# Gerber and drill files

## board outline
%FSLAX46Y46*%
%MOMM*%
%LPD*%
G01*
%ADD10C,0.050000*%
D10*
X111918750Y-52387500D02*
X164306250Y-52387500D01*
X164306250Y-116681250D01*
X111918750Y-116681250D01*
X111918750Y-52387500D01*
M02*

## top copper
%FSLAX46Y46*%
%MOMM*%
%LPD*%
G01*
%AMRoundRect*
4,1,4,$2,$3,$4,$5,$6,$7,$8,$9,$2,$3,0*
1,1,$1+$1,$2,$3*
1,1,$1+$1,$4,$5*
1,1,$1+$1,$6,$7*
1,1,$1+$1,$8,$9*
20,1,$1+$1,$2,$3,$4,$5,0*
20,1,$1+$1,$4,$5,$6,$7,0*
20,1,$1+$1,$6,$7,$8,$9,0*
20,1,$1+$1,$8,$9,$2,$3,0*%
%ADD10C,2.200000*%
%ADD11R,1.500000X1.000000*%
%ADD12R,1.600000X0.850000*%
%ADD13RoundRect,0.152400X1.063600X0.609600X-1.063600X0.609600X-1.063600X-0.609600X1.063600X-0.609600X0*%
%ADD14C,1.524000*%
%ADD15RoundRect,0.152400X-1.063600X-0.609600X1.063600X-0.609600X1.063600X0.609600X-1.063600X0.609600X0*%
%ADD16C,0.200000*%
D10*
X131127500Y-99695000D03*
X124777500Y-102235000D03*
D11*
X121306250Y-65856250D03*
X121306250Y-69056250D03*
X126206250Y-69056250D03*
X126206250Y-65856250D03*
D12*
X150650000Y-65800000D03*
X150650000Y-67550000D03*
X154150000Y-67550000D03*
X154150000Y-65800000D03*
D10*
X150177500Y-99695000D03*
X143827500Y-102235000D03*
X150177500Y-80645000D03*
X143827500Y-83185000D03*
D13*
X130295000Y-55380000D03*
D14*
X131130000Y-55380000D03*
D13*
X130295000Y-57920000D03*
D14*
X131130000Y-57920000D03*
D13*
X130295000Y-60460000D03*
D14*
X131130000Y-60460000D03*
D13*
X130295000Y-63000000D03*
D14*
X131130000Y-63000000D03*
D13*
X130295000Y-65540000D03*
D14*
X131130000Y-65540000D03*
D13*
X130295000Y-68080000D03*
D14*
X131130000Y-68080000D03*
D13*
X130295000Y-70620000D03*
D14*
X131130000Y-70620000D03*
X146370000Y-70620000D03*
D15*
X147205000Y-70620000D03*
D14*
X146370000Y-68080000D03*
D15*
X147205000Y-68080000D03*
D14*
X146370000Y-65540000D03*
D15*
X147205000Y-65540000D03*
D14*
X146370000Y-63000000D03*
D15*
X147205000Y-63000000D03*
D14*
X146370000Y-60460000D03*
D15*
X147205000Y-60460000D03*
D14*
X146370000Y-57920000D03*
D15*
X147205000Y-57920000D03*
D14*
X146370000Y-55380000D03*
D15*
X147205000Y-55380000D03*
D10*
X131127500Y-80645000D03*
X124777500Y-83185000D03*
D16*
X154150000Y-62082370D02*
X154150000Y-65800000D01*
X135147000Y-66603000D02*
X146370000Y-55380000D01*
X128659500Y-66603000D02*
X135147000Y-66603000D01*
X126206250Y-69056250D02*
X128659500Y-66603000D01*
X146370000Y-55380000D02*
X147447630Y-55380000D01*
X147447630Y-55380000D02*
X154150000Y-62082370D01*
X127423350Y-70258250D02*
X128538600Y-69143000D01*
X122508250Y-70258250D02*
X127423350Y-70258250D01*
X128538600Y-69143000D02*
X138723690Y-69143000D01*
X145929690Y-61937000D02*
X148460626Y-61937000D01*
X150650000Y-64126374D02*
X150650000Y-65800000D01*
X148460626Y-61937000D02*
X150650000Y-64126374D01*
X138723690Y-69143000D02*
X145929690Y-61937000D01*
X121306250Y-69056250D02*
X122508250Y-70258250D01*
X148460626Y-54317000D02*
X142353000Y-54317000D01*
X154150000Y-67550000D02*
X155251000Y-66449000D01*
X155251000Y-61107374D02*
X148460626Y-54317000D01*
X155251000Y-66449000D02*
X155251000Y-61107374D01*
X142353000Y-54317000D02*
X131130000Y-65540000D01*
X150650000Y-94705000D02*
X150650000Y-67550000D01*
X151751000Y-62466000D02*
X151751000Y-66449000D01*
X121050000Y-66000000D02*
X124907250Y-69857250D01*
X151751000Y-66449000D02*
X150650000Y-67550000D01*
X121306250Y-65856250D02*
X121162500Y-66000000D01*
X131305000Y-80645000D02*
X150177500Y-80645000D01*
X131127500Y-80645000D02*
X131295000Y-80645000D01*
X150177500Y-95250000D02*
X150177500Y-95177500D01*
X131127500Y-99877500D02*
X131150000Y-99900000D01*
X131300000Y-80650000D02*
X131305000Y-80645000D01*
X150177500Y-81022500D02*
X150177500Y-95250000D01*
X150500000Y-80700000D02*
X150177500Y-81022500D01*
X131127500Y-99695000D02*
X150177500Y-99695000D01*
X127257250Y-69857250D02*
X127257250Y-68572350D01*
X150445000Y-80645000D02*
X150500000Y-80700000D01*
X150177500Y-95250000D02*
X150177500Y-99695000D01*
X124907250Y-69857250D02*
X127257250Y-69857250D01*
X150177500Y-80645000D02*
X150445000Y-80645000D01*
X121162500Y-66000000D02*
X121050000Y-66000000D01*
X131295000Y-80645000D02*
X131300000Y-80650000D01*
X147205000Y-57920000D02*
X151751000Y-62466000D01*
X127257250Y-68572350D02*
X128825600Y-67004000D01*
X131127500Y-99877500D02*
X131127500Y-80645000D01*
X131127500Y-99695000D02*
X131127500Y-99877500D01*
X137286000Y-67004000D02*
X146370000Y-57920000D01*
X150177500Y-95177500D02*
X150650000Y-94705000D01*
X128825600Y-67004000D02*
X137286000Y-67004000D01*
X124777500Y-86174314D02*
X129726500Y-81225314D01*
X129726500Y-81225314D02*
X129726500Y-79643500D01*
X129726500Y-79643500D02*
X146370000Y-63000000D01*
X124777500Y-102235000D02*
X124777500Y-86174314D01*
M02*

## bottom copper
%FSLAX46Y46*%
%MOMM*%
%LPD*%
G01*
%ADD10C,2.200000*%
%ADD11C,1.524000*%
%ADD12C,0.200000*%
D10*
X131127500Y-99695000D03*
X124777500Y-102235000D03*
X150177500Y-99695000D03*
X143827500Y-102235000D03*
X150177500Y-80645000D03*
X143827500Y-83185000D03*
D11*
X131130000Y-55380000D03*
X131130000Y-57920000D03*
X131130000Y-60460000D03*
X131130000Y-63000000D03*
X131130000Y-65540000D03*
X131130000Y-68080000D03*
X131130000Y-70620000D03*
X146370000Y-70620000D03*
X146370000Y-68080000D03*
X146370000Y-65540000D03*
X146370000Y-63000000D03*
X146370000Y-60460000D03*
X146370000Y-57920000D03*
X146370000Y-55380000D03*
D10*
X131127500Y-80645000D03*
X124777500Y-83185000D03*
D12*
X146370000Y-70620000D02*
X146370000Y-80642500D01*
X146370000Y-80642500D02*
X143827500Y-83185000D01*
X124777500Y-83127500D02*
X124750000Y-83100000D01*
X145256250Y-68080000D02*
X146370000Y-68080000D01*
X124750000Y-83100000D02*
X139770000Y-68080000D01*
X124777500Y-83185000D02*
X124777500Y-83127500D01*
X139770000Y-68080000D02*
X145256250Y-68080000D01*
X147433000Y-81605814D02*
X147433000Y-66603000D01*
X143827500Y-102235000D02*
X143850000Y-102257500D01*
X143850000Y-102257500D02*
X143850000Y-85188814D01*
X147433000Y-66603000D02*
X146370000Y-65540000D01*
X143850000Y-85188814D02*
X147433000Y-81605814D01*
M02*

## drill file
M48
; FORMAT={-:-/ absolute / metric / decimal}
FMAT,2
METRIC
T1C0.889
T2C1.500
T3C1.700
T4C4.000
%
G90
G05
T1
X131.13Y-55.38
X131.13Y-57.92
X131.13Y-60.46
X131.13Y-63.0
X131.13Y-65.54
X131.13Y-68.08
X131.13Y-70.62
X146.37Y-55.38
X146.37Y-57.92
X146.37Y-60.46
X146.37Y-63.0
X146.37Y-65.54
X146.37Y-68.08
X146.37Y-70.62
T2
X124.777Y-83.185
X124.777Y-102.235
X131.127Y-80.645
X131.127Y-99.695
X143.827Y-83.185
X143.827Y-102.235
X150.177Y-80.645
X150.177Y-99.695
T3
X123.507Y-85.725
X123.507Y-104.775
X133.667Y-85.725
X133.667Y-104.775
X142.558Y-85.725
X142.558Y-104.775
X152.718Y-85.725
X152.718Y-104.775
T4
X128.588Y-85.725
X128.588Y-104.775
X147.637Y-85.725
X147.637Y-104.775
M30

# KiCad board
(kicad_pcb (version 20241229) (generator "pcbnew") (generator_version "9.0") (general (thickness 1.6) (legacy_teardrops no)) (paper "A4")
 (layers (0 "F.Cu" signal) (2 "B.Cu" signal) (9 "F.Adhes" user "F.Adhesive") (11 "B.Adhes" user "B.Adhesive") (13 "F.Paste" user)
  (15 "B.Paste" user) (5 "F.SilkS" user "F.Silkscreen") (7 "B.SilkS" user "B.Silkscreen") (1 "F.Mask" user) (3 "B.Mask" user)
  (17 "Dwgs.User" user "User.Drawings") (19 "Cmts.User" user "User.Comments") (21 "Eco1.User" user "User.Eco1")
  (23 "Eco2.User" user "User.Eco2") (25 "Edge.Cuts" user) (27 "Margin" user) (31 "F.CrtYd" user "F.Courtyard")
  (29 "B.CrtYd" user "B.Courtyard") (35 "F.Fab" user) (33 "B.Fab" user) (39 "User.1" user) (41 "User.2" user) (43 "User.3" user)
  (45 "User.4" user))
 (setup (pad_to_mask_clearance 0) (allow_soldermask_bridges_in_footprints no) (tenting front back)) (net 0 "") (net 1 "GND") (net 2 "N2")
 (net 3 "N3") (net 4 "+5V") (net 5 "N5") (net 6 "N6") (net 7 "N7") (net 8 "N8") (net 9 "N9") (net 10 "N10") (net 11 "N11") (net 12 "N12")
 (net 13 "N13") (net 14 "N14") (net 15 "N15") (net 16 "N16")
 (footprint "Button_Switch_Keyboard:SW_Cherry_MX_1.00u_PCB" (layer "F.Cu") (at 131.1275 99.695)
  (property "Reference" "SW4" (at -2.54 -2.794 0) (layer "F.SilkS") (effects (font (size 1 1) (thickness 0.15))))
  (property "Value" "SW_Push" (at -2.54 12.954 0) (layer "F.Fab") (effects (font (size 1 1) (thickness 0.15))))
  (pad "" np_thru_hole circle (at -7.62 5.08) (size 1.7 1.7) (drill 1.7) (layers "*.Cu" "*.Mask"))
  (pad "" np_thru_hole circle (at -2.54 5.08) (size 4 4) (drill 4) (layers "*.Cu" "*.Mask"))
  (pad "" np_thru_hole circle (at 2.54 5.08) (size 1.7 1.7) (drill 1.7) (layers "*.Cu" "*.Mask"))
  (pad "1" thru_hole circle (at 0 0) (size 2.2 2.2) (drill 1.5) (layers "*.Cu" "*.Mask") (remove_unused_layers no) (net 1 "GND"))
  (pad "2" thru_hole circle (at -6.35 2.54) (size 2.2 2.2) (drill 1.5) (layers "*.Cu" "*.Mask") (remove_unused_layers no) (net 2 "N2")))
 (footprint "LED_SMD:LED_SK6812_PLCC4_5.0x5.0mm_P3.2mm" (layer "F.Cu") (at 123.75625 67.45625)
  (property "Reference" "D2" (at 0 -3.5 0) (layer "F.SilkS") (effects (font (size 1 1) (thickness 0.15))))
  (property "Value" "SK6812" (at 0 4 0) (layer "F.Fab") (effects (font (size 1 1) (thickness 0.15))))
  (pad "1" smd rect (at -2.45 -1.6 180) (size 1.5 1) (layers "F.Cu" "F.Mask" "F.Paste") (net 1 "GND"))
  (pad "2" smd rect (at -2.45 1.6 180) (size 1.5 1) (layers "F.Cu" "F.Mask" "F.Paste") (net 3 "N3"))
  (pad "3" smd rect (at 2.45 1.6 180) (size 1.5 1) (layers "F.Cu" "F.Mask" "F.Paste") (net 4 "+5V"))
  (pad "4" smd rect (at 2.45 -1.6 180) (size 1.5 1) (layers "F.Cu" "F.Mask" "F.Paste") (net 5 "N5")))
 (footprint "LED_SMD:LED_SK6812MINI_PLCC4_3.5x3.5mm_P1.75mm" (layer "F.Cu") (at 152.4 66.675)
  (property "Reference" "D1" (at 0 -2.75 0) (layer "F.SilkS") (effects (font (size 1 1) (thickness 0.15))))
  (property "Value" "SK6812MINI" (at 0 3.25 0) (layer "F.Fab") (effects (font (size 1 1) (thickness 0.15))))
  (pad "1" smd rect (at -1.75 -0.875) (size 1.6 0.85) (layers "F.Cu" "F.Mask" "F.Paste") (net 3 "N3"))
  (pad "2" smd rect (at -1.75 0.875) (size 1.6 0.85) (layers "F.Cu" "F.Mask" "F.Paste") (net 1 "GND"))
  (pad "3" smd rect (at 1.75 0.875) (size 1.6 0.85) (layers "F.Cu" "F.Mask" "F.Paste") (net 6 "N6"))
  (pad "4" smd rect (at 1.75 -0.875) (size 1.6 0.85) (layers "F.Cu" "F.Mask" "F.Paste") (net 4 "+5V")))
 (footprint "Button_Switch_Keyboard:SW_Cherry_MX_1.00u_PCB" (layer "F.Cu") (at 150.1775 99.695)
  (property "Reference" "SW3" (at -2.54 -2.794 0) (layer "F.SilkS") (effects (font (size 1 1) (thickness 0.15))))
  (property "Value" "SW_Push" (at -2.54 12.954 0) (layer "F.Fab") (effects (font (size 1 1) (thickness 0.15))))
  (pad "" np_thru_hole circle (at -7.62 5.08) (size 1.7 1.7) (drill 1.7) (layers "*.Cu" "*.Mask"))
  (pad "" np_thru_hole circle (at -2.54 5.08) (size 4 4) (drill 4) (layers "*.Cu" "*.Mask"))
  (pad "" np_thru_hole circle (at 2.54 5.08) (size 1.7 1.7) (drill 1.7) (layers "*.Cu" "*.Mask"))
  (pad "1" thru_hole circle (at 0 0) (size 2.2 2.2) (drill 1.5) (layers "*.Cu" "*.Mask") (remove_unused_layers no) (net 1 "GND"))
  (pad "2" thru_hole circle (at -6.35 2.54) (size 2.2 2.2) (drill 1.5) (layers "*.Cu" "*.Mask") (remove_unused_layers no) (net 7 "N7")))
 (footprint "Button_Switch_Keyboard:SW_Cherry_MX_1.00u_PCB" (layer "F.Cu") (at 150.1775 80.645)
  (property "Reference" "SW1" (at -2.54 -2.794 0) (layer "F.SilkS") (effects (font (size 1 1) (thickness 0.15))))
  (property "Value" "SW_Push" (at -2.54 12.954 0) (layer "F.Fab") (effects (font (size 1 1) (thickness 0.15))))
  (pad "" np_thru_hole circle (at -7.62 5.08) (size 1.7 1.7) (drill 1.7) (layers "*.Cu" "*.Mask"))
  (pad "" np_thru_hole circle (at -2.54 5.08) (size 4 4) (drill 4) (layers "*.Cu" "*.Mask"))
  (pad "" np_thru_hole circle (at 2.54 5.08) (size 1.7 1.7) (drill 1.7) (layers "*.Cu" "*.Mask"))
  (pad "1" thru_hole circle (at 0 0) (size 2.2 2.2) (drill 1.5) (layers "*.Cu" "*.Mask") (remove_unused_layers no) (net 1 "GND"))
  (pad "2" thru_hole circle (at -6.35 2.54) (size 2.2 2.2) (drill 1.5) (layers "*.Cu" "*.Mask") (remove_unused_layers no) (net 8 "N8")))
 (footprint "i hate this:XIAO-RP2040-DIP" (layer "F.Cu") (at 138.75 63)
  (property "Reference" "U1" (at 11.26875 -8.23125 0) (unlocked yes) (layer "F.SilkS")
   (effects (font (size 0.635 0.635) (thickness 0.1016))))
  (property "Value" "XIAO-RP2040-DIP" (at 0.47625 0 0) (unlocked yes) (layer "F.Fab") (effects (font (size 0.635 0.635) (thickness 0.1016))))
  (pad "1" smd roundrect (at -8.455 -7.62 180) (size 2.432 1.524) (layers "F.Cu" "F.Mask") (roundrect_rratio 0.1) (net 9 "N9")
   (thermal_bridge_angle 45))
  (pad "1" thru_hole circle (at -7.62 -7.62 180) (size 1.524 1.524) (drill 0.889) (layers "*.Cu" "*.Mask") (remove_unused_layers no)
   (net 9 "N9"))
  (pad "2" smd roundrect (at -8.455 -5.08 180) (size 2.432 1.524) (layers "F.Cu" "F.Mask") (roundrect_rratio 0.1) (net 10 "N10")
   (thermal_bridge_angle 45))
  (pad "2" thru_hole circle (at -7.62 -5.08 180) (size 1.524 1.524) (drill 0.889) (layers "*.Cu" "*.Mask") (remove_unused_layers no)
   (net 10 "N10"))
  (pad "3" smd roundrect (at -8.455 -2.54 180) (size 2.432 1.524) (layers "F.Cu" "F.Mask") (roundrect_rratio 0.1) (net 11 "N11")
   (thermal_bridge_angle 45))
  (pad "3" thru_hole circle (at -7.62 -2.54 180) (size 1.524 1.524) (drill 0.889) (layers "*.Cu" "*.Mask") (remove_unused_layers no)
   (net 11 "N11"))
  (pad "4" smd roundrect (at -8.455 0 180) (size 2.432 1.524) (layers "F.Cu" "F.Mask") (roundrect_rratio 0.1) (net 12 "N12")
   (thermal_bridge_angle 45))
  (pad "4" thru_hole circle (at -7.62 0 180) (size 1.524 1.524) (drill 0.889) (layers "*.Cu" "*.Mask") (remove_unused_layers no)
   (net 12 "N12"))
  (pad "5" smd roundrect (at -8.455 2.54 180) (size 2.432 1.524) (layers "F.Cu" "F.Mask") (roundrect_rratio 0.1) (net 6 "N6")
   (thermal_bridge_angle 45))
  (pad "5" thru_hole circle (at -7.62 2.54 180) (size 1.524 1.524) (drill 0.889) (layers "*.Cu" "*.Mask") (remove_unused_layers no)
   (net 6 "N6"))
  (pad "6" smd roundrect (at -8.455 5.08 180) (size 2.432 1.524) (layers "F.Cu" "F.Mask") (roundrect_rratio 0.1) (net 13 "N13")
   (thermal_bridge_angle 45))
  (pad "6" thru_hole circle (at -7.62 5.08 180) (size 1.524 1.524) (drill 0.889) (layers "*.Cu" "*.Mask") (remove_unused_layers no)
   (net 13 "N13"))
  (pad "7" smd roundrect (at -8.455 7.62 180) (size 2.432 1.524) (layers "F.Cu" "F.Mask") (roundrect_rratio 0.1) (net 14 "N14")
   (thermal_bridge_angle 45))
  (pad "7" thru_hole circle (at -7.62 7.62 180) (size 1.524 1.524) (drill 0.889) (layers "*.Cu" "*.Mask") (remove_unused_layers no)
   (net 14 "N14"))
  (pad "8" thru_hole circle (at 7.62 7.62) (size 1.524 1.524) (drill 0.889) (layers "*.Cu" "*.Mask") (remove_unused_layers no) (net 8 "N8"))
  (pad "8" smd roundrect (at 8.455 7.62) (size 2.432 1.524) (layers "F.Cu" "F.Mask") (roundrect_rratio 0.1) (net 8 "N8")
   (thermal_bridge_angle 45))
  (pad "9" thru_hole circle (at 7.62 5.08) (size 1.524 1.524) (drill 0.889) (layers "*.Cu" "*.Mask") (remove_unused_layers no)
   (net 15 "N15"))
  (pad "9" smd roundrect (at 8.455 5.08) (size 2.432 1.524) (layers "F.Cu" "F.Mask") (roundrect_rratio 0.1) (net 15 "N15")
   (thermal_bridge_angle 45))
  (pad "10" thru_hole circle (at 7.62 2.54) (size 1.524 1.524) (drill 0.889) (layers "*.Cu" "*.Mask") (remove_unused_layers no) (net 7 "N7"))
  (pad "10" smd roundrect (at 8.455 2.54) (size 2.432 1.524) (layers "F.Cu" "F.Mask") (roundrect_rratio 0.1) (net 7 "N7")
   (thermal_bridge_angle 45))
  (pad "11" thru_hole circle (at 7.62 0) (size 1.524 1.524) (drill 0.889) (layers "*.Cu" "*.Mask") (remove_unused_layers no) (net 2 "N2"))
  (pad "11" smd roundrect (at 8.455 0) (size 2.432 1.524) (layers "F.Cu" "F.Mask") (roundrect_rratio 0.1) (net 2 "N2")
   (thermal_bridge_angle 45))
  (pad "12" thru_hole circle (at 7.62 -2.54) (size 1.524 1.524) (drill 0.889) (layers "*.Cu" "*.Mask") (remove_unused_layers no)
   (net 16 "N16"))
  (pad "12" smd roundrect (at 8.455 -2.54) (size 2.432 1.524) (layers "F.Cu" "F.Mask") (roundrect_rratio 0.1) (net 16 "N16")
   (thermal_bridge_angle 45))
  (pad "13" thru_hole circle (at 7.62 -5.08) (size 1.524 1.524) (drill 0.889) (layers "*.Cu" "*.Mask") (remove_unused_layers no)
   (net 1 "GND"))
  (pad "13" smd roundrect (at 8.455 -5.08) (size 2.432 1.524) (layers "F.Cu" "F.Mask") (roundrect_rratio 0.1) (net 1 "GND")
   (thermal_bridge_angle 45))
  (pad "14" thru_hole circle (at 7.62 -7.62) (size 1.524 1.524) (drill 0.889) (layers "*.Cu" "*.Mask") (remove_unused_layers no)
   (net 4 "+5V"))
  (pad "14" smd roundrect (at 8.455 -7.62) (size 2.432 1.524) (layers "F.Cu" "F.Mask") (roundrect_rratio 0.1) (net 4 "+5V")
   (thermal_bridge_angle 45)))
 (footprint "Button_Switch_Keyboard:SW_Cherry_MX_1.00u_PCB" (layer "F.Cu") (at 131.1275 80.645)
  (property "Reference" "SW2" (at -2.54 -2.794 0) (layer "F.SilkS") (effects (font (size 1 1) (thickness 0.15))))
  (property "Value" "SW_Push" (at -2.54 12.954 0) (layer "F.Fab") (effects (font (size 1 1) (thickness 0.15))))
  (pad "" np_thru_hole circle (at -7.62 5.08) (size 1.7 1.7) (drill 1.7) (layers "*.Cu" "*.Mask"))
  (pad "" np_thru_hole circle (at -2.54 5.08) (size 4 4) (drill 4) (layers "*.Cu" "*.Mask"))
  (pad "" np_thru_hole circle (at 2.54 5.08) (size 1.7 1.7) (drill 1.7) (layers "*.Cu" "*.Mask"))
  (pad "1" thru_hole circle (at 0 0) (size 2.2 2.2) (drill 1.5) (layers "*.Cu" "*.Mask") (remove_unused_layers no) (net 1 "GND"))
  (pad "2" thru_hole circle (at -6.35 2.54) (size 2.2 2.2) (drill 1.5) (layers "*.Cu" "*.Mask") (remove_unused_layers no) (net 15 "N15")))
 (gr_rect (start 111.91875 52.3875) (end 164.30625 116.68125) (stroke (width 0.05) (type default)) (fill no) (layer "Edge.Cuts"))
 (segment (start 154.15 62.08237) (end 154.15 65.8) (width 0.2) (layer "F.Cu") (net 4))
 (segment (start 135.147 66.603) (end 146.37 55.38) (width 0.2) (layer "F.Cu") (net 4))
 (segment (start 128.6595 66.603) (end 135.147 66.603) (width 0.2) (layer "F.Cu") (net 4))
 (segment (start 126.20625 69.05625) (end 128.6595 66.603) (width 0.2) (layer "F.Cu") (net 4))
 (segment (start 146.37 55.38) (end 147.44763 55.38) (width 0.2) (layer "F.Cu") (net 4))
 (segment (start 147.44763 55.38) (end 154.15 62.08237) (width 0.2) (layer "F.Cu") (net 4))
 (segment (start 127.42335 70.25825) (end 128.5386 69.143) (width 0.2) (layer "F.Cu") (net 3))
 (segment (start 122.50825 70.25825) (end 127.42335 70.25825) (width 0.2) (layer "F.Cu") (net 3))
 (segment (start 128.5386 69.143) (end 138.72369 69.143) (width 0.2) (layer "F.Cu") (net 3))
 (segment (start 145.92969 61.937) (end 148.460626 61.937) (width 0.2) (layer "F.Cu") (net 3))
 (segment (start 150.65 64.126374) (end 150.65 65.8) (width 0.2) (layer "F.Cu") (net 3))
 (segment (start 148.460626 61.937) (end 150.65 64.126374) (width 0.2) (layer "F.Cu") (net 3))
 (segment (start 138.72369 69.143) (end 145.92969 61.937) (width 0.2) (layer "F.Cu") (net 3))
 (segment (start 121.30625 69.05625) (end 122.50825 70.25825) (width 0.2) (layer "F.Cu") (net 3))
 (segment (start 148.460626 54.317) (end 142.353 54.317) (width 0.2) (layer "F.Cu") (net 6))
 (segment (start 154.15 67.55) (end 155.251 66.449) (width 0.2) (layer "F.Cu") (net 6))
 (segment (start 155.251 61.107374) (end 148.460626 54.317) (width 0.2) (layer "F.Cu") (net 6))
 (segment (start 155.251 66.449) (end 155.251 61.107374) (width 0.2) (layer "F.Cu") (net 6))
 (segment (start 142.353 54.317) (end 131.13 65.54) (width 0.2) (layer "F.Cu") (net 6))
 (segment (start 150.65 94.705) (end 150.65 67.55) (width 0.2) (layer "F.Cu") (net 1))
 (segment (start 151.751 62.466) (end 151.751 66.449) (width 0.2) (layer "F.Cu") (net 1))
 (segment (start 121.05 66) (end 124.90725 69.85725) (width 0.2) (layer "F.Cu") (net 1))
 (segment (start 151.751 66.449) (end 150.65 67.55) (width 0.2) (layer "F.Cu") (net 1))
 (segment (start 121.30625 65.85625) (end 121.1625 66) (width 0.2) (layer "F.Cu") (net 1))
 (segment (start 131.305 80.645) (end 150.1775 80.645) (width 0.2) (layer "F.Cu") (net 1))
 (segment (start 131.1275 80.645) (end 131.295 80.645) (width 0.2) (layer "F.Cu") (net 1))
 (segment (start 150.1775 95.25) (end 150.1775 95.1775) (width 0.2) (layer "F.Cu") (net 1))
 (segment (start 131.1275 99.8775) (end 131.15 99.9) (width 0.2) (layer "F.Cu") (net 1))
 (segment (start 131.3 80.65) (end 131.305 80.645) (width 0.2) (layer "F.Cu") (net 1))
 (segment (start 150.1775 81.0225) (end 150.1775 95.25) (width 0.2) (layer "F.Cu") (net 1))
 (segment (start 150.5 80.7) (end 150.1775 81.0225) (width 0.2) (layer "F.Cu") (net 1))
 (segment (start 131.1275 99.695) (end 150.1775 99.695) (width 0.2) (layer "F.Cu") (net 1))
 (segment (start 127.25725 69.85725) (end 127.25725 68.57235) (width 0.2) (layer "F.Cu") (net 1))
 (segment (start 150.445 80.645) (end 150.5 80.7) (width 0.2) (layer "F.Cu") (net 1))
 (segment (start 150.1775 95.25) (end 150.1775 99.695) (width 0.2) (layer "F.Cu") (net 1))
 (segment (start 124.90725 69.85725) (end 127.25725 69.85725) (width 0.2) (layer "F.Cu") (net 1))
 (segment (start 150.1775 80.645) (end 150.445 80.645) (width 0.2) (layer "F.Cu") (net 1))
 (segment (start 121.1625 66) (end 121.05 66) (width 0.2) (layer "F.Cu") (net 1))
 (segment (start 131.295 80.645) (end 131.3 80.65) (width 0.2) (layer "F.Cu") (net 1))
 (segment (start 147.205 57.92) (end 151.751 62.466) (width 0.2) (layer "F.Cu") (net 1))
 (segment (start 127.25725 68.57235) (end 128.8256 67.004) (width 0.2) (layer "F.Cu") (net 1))
 (segment (start 131.1275 99.8775) (end 131.1275 80.645) (width 0.2) (layer "F.Cu") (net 1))
 (segment (start 131.1275 99.695) (end 131.1275 99.8775) (width 0.2) (layer "F.Cu") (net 1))
 (segment (start 137.286 67.004) (end 146.37 57.92) (width 0.2) (layer "F.Cu") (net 1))
 (segment (start 150.1775 95.1775) (end 150.65 94.705) (width 0.2) (layer "F.Cu") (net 1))
 (segment (start 128.8256 67.004) (end 137.286 67.004) (width 0.2) (layer "F.Cu") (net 1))
 (segment (start 146.37 70.62) (end 146.37 80.6425) (width 0.2) (layer "B.Cu") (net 8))
 (segment (start 146.37 80.6425) (end 143.8275 83.185) (width 0.2) (layer "B.Cu") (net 8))
 (segment (start 124.7775 83.1275) (end 124.75 83.1) (width 0.2) (layer "B.Cu") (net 15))
 (segment (start 145.25625 68.08) (end 146.37 68.08) (width 0.2) (layer "B.Cu") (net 15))
 (segment (start 124.75 83.1) (end 139.77 68.08) (width 0.2) (layer "B.Cu") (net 15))
 (segment (start 124.7775 83.185) (end 124.7775 83.1275) (width 0.2) (layer "B.Cu") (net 15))
 (segment (start 139.77 68.08) (end 145.25625 68.08) (width 0.2) (layer "B.Cu") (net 15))
 (segment (start 147.433 81.605814) (end 147.433 66.603) (width 0.2) (layer "B.Cu") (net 7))
 (segment (start 143.8275 102.235) (end 143.85 102.2575) (width 0.2) (layer "B.Cu") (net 7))
 (segment (start 143.85 102.2575) (end 143.85 85.188814) (width 0.2) (layer "B.Cu") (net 7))
 (segment (start 147.433 66.603) (end 146.37 65.54) (width 0.2) (layer "B.Cu") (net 7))
 (segment (start 143.85 85.188814) (end 147.433 81.605814) (width 0.2) (layer "B.Cu") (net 7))
 (segment (start 124.7775 86.174314) (end 129.7265 81.225314) (width 0.2) (layer "F.Cu") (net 2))
 (segment (start 129.7265 81.225314) (end 129.7265 79.6435) (width 0.2) (layer "F.Cu") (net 2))
 (segment (start 129.7265 79.6435) (end 146.37 63) (width 0.2) (layer "F.Cu") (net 2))
 (segment (start 124.7775 102.235) (end 124.7775 86.174314) (width 0.2) (layer "F.Cu") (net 2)))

